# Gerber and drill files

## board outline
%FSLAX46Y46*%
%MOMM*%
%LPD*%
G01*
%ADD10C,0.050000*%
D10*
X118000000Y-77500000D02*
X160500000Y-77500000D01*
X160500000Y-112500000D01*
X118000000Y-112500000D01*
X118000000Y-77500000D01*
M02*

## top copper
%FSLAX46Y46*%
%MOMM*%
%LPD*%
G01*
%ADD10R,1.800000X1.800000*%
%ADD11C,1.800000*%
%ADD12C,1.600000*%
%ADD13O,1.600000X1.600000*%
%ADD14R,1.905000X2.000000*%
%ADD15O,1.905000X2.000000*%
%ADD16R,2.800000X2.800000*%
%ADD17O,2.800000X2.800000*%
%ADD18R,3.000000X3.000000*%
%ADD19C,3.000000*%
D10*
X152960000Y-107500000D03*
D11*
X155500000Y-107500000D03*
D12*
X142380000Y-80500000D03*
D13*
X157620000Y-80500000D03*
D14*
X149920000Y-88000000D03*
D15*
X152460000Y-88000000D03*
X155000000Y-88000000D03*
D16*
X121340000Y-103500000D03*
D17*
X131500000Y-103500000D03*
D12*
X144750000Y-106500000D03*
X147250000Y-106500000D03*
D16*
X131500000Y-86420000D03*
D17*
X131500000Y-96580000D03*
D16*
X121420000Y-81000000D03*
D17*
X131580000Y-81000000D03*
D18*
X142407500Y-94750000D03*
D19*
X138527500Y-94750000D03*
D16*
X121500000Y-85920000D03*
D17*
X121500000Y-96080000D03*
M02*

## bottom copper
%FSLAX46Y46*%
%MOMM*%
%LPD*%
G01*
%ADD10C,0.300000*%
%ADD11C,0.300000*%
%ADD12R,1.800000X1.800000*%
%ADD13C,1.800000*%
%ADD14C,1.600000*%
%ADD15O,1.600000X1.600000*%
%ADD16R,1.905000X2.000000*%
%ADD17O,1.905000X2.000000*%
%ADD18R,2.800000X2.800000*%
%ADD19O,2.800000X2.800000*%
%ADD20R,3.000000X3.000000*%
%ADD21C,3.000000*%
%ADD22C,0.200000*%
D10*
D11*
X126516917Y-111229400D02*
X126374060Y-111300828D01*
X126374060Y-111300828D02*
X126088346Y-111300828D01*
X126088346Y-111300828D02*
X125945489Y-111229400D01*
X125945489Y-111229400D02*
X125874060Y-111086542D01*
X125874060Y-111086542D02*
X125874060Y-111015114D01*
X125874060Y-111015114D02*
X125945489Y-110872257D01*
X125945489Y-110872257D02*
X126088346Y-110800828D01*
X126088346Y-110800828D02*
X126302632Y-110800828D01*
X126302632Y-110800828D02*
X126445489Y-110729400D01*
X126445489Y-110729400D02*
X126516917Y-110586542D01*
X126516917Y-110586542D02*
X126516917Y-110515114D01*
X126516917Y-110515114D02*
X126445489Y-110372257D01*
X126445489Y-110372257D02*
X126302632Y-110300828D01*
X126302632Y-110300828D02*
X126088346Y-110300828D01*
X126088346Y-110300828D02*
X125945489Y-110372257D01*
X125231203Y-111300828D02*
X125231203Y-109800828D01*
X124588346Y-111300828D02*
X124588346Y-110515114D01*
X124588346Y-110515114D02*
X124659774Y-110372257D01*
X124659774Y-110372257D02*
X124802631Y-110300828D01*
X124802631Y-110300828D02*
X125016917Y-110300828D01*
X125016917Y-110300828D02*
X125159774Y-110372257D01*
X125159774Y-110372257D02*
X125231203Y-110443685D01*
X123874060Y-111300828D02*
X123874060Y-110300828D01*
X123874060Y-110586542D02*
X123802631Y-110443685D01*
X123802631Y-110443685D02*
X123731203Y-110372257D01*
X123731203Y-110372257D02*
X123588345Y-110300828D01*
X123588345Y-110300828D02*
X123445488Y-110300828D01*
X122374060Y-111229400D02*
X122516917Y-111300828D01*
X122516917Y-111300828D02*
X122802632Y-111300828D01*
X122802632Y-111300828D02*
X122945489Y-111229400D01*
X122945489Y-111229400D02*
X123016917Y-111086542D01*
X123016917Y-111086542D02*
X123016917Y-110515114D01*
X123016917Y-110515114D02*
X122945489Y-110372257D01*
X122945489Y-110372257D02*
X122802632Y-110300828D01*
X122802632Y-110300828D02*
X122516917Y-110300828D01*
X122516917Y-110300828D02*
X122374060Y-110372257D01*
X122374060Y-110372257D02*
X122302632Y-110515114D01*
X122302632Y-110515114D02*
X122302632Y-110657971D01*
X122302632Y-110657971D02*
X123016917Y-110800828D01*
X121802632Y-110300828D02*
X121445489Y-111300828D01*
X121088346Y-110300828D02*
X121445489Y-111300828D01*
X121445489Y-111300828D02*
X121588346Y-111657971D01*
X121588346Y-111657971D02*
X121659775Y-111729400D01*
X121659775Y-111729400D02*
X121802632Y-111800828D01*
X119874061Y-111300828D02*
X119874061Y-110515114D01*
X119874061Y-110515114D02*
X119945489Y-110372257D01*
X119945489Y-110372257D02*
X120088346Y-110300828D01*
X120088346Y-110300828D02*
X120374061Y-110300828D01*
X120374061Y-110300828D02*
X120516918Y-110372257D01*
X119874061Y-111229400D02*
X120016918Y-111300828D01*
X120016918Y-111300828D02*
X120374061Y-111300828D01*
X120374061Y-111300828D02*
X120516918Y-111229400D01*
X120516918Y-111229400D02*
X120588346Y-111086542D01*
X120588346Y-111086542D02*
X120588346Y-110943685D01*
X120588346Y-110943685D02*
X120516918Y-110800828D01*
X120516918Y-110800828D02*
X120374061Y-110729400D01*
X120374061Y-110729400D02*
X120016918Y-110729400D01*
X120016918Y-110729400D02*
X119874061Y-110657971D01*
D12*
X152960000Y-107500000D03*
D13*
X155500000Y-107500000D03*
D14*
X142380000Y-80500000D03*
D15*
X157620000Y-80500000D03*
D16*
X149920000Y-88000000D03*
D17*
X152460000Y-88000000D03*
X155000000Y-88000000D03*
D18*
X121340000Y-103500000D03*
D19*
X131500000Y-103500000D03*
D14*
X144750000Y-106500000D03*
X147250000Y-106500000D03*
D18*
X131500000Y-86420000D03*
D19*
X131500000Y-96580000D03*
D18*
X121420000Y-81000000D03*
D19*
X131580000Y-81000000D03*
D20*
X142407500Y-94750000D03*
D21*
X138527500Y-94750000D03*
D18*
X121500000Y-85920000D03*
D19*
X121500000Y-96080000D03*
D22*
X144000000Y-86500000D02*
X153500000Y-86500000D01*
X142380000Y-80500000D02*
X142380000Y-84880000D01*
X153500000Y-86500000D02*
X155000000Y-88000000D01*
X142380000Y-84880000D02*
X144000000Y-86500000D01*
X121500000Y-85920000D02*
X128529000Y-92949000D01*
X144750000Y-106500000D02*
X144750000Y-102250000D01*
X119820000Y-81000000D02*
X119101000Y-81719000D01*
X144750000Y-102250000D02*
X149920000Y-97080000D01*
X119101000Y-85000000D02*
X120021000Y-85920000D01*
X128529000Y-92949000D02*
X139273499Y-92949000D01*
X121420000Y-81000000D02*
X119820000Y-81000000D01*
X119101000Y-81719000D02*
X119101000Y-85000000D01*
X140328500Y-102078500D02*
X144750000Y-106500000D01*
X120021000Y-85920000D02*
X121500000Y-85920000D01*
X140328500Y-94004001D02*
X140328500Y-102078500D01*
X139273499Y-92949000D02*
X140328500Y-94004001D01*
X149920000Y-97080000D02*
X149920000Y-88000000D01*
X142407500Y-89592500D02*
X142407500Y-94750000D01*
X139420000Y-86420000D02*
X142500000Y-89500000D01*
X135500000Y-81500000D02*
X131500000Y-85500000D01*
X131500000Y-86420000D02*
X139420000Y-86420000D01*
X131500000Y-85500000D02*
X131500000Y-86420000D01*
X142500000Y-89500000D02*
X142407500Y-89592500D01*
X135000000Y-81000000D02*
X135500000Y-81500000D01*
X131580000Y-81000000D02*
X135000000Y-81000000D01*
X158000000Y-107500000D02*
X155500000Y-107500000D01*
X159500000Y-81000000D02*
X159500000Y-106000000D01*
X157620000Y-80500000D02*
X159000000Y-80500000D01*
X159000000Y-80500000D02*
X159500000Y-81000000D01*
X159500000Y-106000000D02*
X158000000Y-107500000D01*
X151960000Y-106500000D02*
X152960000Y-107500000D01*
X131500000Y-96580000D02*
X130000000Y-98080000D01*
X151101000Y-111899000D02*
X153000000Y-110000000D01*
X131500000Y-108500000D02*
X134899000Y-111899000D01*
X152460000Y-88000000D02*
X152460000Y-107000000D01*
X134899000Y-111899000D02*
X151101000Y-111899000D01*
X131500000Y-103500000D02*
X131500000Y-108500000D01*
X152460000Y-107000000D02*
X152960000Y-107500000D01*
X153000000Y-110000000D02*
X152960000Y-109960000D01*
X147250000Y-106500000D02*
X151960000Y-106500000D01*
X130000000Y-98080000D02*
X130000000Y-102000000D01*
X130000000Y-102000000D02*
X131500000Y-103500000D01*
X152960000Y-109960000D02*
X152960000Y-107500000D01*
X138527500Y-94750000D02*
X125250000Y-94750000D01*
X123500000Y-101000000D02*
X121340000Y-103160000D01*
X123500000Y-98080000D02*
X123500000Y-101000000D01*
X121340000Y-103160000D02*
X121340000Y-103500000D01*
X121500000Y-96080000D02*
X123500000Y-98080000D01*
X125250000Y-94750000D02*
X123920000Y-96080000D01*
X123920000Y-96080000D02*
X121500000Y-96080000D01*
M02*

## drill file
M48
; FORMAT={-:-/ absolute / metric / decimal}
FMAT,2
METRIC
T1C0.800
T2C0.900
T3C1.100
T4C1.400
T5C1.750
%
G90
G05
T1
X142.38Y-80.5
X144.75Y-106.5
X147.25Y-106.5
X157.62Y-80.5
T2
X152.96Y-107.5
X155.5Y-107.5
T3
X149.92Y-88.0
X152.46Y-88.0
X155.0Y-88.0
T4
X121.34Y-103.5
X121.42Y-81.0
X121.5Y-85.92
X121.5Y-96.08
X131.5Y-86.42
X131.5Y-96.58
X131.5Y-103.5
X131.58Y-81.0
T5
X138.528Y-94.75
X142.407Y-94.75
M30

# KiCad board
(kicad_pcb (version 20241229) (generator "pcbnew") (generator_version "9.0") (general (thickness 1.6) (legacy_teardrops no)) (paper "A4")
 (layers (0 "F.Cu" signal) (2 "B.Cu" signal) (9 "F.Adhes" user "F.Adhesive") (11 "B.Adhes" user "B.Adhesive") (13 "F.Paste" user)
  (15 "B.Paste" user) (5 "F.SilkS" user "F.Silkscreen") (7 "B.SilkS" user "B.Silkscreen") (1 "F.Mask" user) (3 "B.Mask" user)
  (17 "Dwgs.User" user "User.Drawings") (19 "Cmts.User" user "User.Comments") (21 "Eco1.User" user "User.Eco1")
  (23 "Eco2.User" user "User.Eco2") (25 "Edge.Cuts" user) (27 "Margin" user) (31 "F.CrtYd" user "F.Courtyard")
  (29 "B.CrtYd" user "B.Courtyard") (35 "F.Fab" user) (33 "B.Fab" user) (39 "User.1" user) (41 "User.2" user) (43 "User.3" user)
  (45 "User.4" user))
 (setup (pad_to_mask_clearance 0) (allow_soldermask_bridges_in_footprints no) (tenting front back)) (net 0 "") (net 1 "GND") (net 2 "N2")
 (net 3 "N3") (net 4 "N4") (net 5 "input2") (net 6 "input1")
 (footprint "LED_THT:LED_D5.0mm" (layer "F.Cu") (at 152.96 107.5)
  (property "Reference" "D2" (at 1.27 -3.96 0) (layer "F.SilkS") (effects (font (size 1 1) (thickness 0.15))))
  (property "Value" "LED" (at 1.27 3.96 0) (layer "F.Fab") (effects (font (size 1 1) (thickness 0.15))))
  (pad "1" thru_hole rect (at 0 0) (size 1.8 1.8) (drill 0.9) (layers "*.Cu" "*.Mask") (remove_unused_layers no) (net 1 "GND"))
  (pad "2" thru_hole circle (at 2.54 0) (size 1.8 1.8) (drill 0.9) (layers "*.Cu" "*.Mask") (remove_unused_layers no) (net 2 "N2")))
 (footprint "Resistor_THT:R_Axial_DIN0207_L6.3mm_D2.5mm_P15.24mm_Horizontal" (layer "F.Cu") (at 142.38 80.5)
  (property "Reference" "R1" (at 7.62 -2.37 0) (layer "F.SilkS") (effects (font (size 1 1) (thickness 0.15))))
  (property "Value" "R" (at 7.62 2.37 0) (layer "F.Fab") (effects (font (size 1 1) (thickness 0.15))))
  (pad "1" thru_hole circle (at 0 0) (size 1.6 1.6) (drill 0.8) (layers "*.Cu" "*.Mask") (remove_unused_layers no) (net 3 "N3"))
  (pad "2" thru_hole oval (at 15.24 0) (size 1.6 1.6) (drill 0.8) (layers "*.Cu" "*.Mask") (remove_unused_layers no) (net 2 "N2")))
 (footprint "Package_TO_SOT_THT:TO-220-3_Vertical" (layer "F.Cu") (at 149.92 88)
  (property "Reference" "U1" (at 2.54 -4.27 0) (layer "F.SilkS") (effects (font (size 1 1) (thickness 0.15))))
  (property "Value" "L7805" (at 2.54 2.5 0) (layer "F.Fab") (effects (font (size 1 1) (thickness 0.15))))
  (pad "1" thru_hole rect (at 0 0) (size 1.905 2) (drill 1.1) (layers "*.Cu" "*.Mask") (remove_unused_layers no) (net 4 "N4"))
  (pad "2" thru_hole oval (at 2.54 0) (size 1.905 2) (drill 1.1) (layers "*.Cu" "*.Mask") (remove_unused_layers no) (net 1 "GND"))
  (pad "3" thru_hole oval (at 5.08 0) (size 1.905 2) (drill 1.1) (layers "*.Cu" "*.Mask") (remove_unused_layers no) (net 3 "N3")))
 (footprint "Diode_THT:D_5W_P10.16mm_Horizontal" (layer "F.Cu") (at 121.34 103.5)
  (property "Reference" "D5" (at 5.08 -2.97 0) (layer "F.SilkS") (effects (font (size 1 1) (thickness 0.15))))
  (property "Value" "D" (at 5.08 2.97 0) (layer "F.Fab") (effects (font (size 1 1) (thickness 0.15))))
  (pad "1" thru_hole rect (at 0 0) (size 2.8 2.8) (drill 1.4) (layers "*.Cu" "*.Mask") (remove_unused_layers no) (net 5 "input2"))
  (pad "2" thru_hole oval (at 10.16 0) (size 2.8 2.8) (drill 1.4) (layers "*.Cu" "*.Mask") (remove_unused_layers no) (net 1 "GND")))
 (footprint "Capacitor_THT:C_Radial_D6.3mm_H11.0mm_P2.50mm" (layer "F.Cu") (at 144.75 106.5)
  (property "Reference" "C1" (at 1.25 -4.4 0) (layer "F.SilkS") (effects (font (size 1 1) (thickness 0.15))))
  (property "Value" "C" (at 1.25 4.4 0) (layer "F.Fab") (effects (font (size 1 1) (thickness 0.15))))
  (pad "1" thru_hole circle (at 0 0) (size 1.6 1.6) (drill 0.8) (layers "*.Cu" "*.Mask") (remove_unused_layers no) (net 4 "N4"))
  (pad "2" thru_hole circle (at 2.5 0) (size 1.6 1.6) (drill 0.8) (layers "*.Cu" "*.Mask") (remove_unused_layers no) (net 1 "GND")))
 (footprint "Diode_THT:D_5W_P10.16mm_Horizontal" (layer "F.Cu") (at 131.5 86.42 -90)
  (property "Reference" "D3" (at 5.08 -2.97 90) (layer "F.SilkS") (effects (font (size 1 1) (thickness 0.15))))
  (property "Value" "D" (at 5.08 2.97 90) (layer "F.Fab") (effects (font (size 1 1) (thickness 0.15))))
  (pad "1" thru_hole rect (at 0 0 270) (size 2.8 2.8) (drill 1.4) (layers "*.Cu" "*.Mask") (remove_unused_layers no) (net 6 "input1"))
  (pad "2" thru_hole oval (at 10.16 0 270) (size 2.8 2.8) (drill 1.4) (layers "*.Cu" "*.Mask") (remove_unused_layers no) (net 1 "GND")))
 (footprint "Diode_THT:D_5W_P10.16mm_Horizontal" (layer "F.Cu") (at 121.42 81)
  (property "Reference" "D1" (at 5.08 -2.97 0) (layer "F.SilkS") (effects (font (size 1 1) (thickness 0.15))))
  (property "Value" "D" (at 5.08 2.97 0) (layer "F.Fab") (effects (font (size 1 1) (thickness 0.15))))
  (pad "1" thru_hole rect (at 0 0) (size 2.8 2.8) (drill 1.4) (layers "*.Cu" "*.Mask") (remove_unused_layers no) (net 4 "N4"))
  (pad "2" thru_hole oval (at 10.16 0) (size 2.8 2.8) (drill 1.4) (layers "*.Cu" "*.Mask") (remove_unused_layers no) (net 6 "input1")))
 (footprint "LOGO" (layer "F.Cu") (at 138.5 81.5)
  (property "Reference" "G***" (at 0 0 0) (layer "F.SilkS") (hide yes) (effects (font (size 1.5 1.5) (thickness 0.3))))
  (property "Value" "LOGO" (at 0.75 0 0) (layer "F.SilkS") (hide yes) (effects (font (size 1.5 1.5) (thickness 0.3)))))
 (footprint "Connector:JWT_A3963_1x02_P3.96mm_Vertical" (layer "F.Cu") (at 142.4075 94.75 180)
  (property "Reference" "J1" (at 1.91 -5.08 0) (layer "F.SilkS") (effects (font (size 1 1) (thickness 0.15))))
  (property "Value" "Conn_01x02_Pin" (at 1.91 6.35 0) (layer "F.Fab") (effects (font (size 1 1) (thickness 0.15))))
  (pad "1" thru_hole rect (at 0 0 180) (size 3 3) (drill 1.75) (layers "*.Cu" "*.Mask") (remove_unused_layers no) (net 6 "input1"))
  (pad "2" thru_hole circle (at 3.88 0 180) (size 3 3) (drill 1.75) (layers "*.Cu" "*.Mask") (remove_unused_layers no) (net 5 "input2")))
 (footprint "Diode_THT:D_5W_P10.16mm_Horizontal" (layer "F.Cu") (at 121.5 85.92 -90)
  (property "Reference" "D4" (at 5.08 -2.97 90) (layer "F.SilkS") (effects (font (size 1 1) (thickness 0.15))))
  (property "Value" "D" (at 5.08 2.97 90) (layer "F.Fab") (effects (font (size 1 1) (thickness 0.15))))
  (pad "1" thru_hole rect (at 0 0 270) (size 2.8 2.8) (drill 1.4) (layers "*.Cu" "*.Mask") (remove_unused_layers no) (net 4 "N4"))
  (pad "2" thru_hole oval (at 10.16 0 270) (size 2.8 2.8) (drill 1.4) (layers "*.Cu" "*.Mask") (remove_unused_layers no) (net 5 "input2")))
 (gr_rect (start 118 77.5) (end 160.5 112.5) (stroke (width 0.05) (type default)) (fill no) (layer "Edge.Cuts"))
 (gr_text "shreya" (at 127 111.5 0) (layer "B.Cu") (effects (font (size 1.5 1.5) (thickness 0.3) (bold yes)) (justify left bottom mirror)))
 (segment (start 144 86.5) (end 153.5 86.5) (width 0.2) (layer "B.Cu") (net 3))
 (segment (start 142.38 80.5) (end 142.38 84.88) (width 0.2) (layer "B.Cu") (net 3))
 (segment (start 153.5 86.5) (end 155 88) (width 0.2) (layer "B.Cu") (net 3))
 (segment (start 142.38 84.88) (end 144 86.5) (width 0.2) (layer "B.Cu") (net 3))
 (segment (start 121.5 85.92) (end 128.529 92.949) (width 0.2) (layer "B.Cu") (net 4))
 (segment (start 144.75 106.5) (end 144.75 102.25) (width 0.2) (layer "B.Cu") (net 4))
 (segment (start 119.82 81) (end 119.101 81.719) (width 0.2) (layer "B.Cu") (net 4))
 (segment (start 144.75 102.25) (end 149.92 97.08) (width 0.2) (layer "B.Cu") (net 4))
 (segment (start 119.101 85) (end 120.021 85.92) (width 0.2) (layer "B.Cu") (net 4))
 (segment (start 128.529 92.949) (end 139.273499 92.949) (width 0.2) (layer "B.Cu") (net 4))
 (segment (start 121.42 81) (end 119.82 81) (width 0.2) (layer "B.Cu") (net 4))
 (segment (start 119.101 81.719) (end 119.101 85) (width 0.2) (layer "B.Cu") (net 4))
 (segment (start 140.3285 102.0785) (end 144.75 106.5) (width 0.2) (layer "B.Cu") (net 4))
 (segment (start 120.021 85.92) (end 121.5 85.92) (width 0.2) (layer "B.Cu") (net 4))
 (segment (start 140.3285 94.004001) (end 140.3285 102.0785) (width 0.2) (layer "B.Cu") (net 4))
 (segment (start 139.273499 92.949) (end 140.3285 94.004001) (width 0.2) (layer "B.Cu") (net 4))
 (segment (start 149.92 97.08) (end 149.92 88) (width 0.2) (layer "B.Cu") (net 4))
 (segment (start 142.4075 89.5925) (end 142.4075 94.75) (width 0.2) (layer "B.Cu") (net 6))
 (segment (start 139.42 86.42) (end 142.5 89.5) (width 0.2) (layer "B.Cu") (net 6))
 (segment (start 135.5 81.5) (end 131.5 85.5) (width 0.2) (layer "B.Cu") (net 6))
 (segment (start 131.5 86.42) (end 139.42 86.42) (width 0.2) (layer "B.Cu") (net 6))
 (segment (start 131.5 85.5) (end 131.5 86.42) (width 0.2) (layer "B.Cu") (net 6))
 (segment (start 142.5 89.5) (end 142.4075 89.5925) (width 0.2) (layer "B.Cu") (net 6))
 (segment (start 135 81) (end 135.5 81.5) (width 0.2) (layer "B.Cu") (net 6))
 (segment (start 131.58 81) (end 135 81) (width 0.2) (layer "B.Cu") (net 6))
 (segment (start 158 107.5) (end 155.5 107.5) (width 0.2) (layer "B.Cu") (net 2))
 (segment (start 159.5 81) (end 159.5 106) (width 0.2) (layer "B.Cu") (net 2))
 (segment (start 157.62 80.5) (end 159 80.5) (width 0.2) (layer "B.Cu") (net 2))
 (segment (start 159 80.5) (end 159.5 81) (width 0.2) (layer "B.Cu") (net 2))
 (segment (start 159.5 106) (end 158 107.5) (width 0.2) (layer "B.Cu") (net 2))
 (segment (start 151.96 106.5) (end 152.96 107.5) (width 0.2) (layer "B.Cu") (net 1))
 (segment (start 131.5 96.58) (end 130 98.08) (width 0.2) (layer "B.Cu") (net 1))
 (segment (start 151.101 111.899) (end 153 110) (width 0.2) (layer "B.Cu") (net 1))
 (segment (start 131.5 108.5) (end 134.899 111.899) (width 0.2) (layer "B.Cu") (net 1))
 (segment (start 152.46 88) (end 152.46 107) (width 0.2) (layer "B.Cu") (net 1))
 (segment (start 134.899 111.899) (end 151.101 111.899) (width 0.2) (layer "B.Cu") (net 1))
 (segment (start 131.5 103.5) (end 131.5 108.5) (width 0.2) (layer "B.Cu") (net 1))
 (segment (start 152.46 107) (end 152.96 107.5) (width 0.2) (layer "B.Cu") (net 1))
 (segment (start 153 110) (end 152.96 109.96) (width 0.2) (layer "B.Cu") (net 1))
 (segment (start 147.25 106.5) (end 151.96 106.5) (width 0.2) (layer "B.Cu") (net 1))
 (segment (start 130 98.08) (end 130 102) (width 0.2) (layer "B.Cu") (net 1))
 (segment (start 130 102) (end 131.5 103.5) (width 0.2) (layer "B.Cu") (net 1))
 (segment (start 152.96 109.96) (end 152.96 107.5) (width 0.2) (layer "B.Cu") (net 1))
 (segment (start 138.5275 94.75) (end 125.25 94.75) (width 0.2) (layer "B.Cu") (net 5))
 (segment (start 123.5 101) (end 121.34 103.16) (width 0.2) (layer "B.Cu") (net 5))
 (segment (start 123.5 98.08) (end 123.5 101) (width 0.2) (layer "B.Cu") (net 5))
 (segment (start 121.34 103.16) (end 121.34 103.5) (width 0.2) (layer "B.Cu") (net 5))
 (segment (start 121.5 96.08) (end 123.5 98.08) (width 0.2) (layer "B.Cu") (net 5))
 (segment (start 125.25 94.75) (end 123.92 96.08) (width 0.2) (layer "B.Cu") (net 5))
 (segment (start 123.92 96.08) (end 121.5 96.08) (width 0.2) (layer "B.Cu") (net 5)))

